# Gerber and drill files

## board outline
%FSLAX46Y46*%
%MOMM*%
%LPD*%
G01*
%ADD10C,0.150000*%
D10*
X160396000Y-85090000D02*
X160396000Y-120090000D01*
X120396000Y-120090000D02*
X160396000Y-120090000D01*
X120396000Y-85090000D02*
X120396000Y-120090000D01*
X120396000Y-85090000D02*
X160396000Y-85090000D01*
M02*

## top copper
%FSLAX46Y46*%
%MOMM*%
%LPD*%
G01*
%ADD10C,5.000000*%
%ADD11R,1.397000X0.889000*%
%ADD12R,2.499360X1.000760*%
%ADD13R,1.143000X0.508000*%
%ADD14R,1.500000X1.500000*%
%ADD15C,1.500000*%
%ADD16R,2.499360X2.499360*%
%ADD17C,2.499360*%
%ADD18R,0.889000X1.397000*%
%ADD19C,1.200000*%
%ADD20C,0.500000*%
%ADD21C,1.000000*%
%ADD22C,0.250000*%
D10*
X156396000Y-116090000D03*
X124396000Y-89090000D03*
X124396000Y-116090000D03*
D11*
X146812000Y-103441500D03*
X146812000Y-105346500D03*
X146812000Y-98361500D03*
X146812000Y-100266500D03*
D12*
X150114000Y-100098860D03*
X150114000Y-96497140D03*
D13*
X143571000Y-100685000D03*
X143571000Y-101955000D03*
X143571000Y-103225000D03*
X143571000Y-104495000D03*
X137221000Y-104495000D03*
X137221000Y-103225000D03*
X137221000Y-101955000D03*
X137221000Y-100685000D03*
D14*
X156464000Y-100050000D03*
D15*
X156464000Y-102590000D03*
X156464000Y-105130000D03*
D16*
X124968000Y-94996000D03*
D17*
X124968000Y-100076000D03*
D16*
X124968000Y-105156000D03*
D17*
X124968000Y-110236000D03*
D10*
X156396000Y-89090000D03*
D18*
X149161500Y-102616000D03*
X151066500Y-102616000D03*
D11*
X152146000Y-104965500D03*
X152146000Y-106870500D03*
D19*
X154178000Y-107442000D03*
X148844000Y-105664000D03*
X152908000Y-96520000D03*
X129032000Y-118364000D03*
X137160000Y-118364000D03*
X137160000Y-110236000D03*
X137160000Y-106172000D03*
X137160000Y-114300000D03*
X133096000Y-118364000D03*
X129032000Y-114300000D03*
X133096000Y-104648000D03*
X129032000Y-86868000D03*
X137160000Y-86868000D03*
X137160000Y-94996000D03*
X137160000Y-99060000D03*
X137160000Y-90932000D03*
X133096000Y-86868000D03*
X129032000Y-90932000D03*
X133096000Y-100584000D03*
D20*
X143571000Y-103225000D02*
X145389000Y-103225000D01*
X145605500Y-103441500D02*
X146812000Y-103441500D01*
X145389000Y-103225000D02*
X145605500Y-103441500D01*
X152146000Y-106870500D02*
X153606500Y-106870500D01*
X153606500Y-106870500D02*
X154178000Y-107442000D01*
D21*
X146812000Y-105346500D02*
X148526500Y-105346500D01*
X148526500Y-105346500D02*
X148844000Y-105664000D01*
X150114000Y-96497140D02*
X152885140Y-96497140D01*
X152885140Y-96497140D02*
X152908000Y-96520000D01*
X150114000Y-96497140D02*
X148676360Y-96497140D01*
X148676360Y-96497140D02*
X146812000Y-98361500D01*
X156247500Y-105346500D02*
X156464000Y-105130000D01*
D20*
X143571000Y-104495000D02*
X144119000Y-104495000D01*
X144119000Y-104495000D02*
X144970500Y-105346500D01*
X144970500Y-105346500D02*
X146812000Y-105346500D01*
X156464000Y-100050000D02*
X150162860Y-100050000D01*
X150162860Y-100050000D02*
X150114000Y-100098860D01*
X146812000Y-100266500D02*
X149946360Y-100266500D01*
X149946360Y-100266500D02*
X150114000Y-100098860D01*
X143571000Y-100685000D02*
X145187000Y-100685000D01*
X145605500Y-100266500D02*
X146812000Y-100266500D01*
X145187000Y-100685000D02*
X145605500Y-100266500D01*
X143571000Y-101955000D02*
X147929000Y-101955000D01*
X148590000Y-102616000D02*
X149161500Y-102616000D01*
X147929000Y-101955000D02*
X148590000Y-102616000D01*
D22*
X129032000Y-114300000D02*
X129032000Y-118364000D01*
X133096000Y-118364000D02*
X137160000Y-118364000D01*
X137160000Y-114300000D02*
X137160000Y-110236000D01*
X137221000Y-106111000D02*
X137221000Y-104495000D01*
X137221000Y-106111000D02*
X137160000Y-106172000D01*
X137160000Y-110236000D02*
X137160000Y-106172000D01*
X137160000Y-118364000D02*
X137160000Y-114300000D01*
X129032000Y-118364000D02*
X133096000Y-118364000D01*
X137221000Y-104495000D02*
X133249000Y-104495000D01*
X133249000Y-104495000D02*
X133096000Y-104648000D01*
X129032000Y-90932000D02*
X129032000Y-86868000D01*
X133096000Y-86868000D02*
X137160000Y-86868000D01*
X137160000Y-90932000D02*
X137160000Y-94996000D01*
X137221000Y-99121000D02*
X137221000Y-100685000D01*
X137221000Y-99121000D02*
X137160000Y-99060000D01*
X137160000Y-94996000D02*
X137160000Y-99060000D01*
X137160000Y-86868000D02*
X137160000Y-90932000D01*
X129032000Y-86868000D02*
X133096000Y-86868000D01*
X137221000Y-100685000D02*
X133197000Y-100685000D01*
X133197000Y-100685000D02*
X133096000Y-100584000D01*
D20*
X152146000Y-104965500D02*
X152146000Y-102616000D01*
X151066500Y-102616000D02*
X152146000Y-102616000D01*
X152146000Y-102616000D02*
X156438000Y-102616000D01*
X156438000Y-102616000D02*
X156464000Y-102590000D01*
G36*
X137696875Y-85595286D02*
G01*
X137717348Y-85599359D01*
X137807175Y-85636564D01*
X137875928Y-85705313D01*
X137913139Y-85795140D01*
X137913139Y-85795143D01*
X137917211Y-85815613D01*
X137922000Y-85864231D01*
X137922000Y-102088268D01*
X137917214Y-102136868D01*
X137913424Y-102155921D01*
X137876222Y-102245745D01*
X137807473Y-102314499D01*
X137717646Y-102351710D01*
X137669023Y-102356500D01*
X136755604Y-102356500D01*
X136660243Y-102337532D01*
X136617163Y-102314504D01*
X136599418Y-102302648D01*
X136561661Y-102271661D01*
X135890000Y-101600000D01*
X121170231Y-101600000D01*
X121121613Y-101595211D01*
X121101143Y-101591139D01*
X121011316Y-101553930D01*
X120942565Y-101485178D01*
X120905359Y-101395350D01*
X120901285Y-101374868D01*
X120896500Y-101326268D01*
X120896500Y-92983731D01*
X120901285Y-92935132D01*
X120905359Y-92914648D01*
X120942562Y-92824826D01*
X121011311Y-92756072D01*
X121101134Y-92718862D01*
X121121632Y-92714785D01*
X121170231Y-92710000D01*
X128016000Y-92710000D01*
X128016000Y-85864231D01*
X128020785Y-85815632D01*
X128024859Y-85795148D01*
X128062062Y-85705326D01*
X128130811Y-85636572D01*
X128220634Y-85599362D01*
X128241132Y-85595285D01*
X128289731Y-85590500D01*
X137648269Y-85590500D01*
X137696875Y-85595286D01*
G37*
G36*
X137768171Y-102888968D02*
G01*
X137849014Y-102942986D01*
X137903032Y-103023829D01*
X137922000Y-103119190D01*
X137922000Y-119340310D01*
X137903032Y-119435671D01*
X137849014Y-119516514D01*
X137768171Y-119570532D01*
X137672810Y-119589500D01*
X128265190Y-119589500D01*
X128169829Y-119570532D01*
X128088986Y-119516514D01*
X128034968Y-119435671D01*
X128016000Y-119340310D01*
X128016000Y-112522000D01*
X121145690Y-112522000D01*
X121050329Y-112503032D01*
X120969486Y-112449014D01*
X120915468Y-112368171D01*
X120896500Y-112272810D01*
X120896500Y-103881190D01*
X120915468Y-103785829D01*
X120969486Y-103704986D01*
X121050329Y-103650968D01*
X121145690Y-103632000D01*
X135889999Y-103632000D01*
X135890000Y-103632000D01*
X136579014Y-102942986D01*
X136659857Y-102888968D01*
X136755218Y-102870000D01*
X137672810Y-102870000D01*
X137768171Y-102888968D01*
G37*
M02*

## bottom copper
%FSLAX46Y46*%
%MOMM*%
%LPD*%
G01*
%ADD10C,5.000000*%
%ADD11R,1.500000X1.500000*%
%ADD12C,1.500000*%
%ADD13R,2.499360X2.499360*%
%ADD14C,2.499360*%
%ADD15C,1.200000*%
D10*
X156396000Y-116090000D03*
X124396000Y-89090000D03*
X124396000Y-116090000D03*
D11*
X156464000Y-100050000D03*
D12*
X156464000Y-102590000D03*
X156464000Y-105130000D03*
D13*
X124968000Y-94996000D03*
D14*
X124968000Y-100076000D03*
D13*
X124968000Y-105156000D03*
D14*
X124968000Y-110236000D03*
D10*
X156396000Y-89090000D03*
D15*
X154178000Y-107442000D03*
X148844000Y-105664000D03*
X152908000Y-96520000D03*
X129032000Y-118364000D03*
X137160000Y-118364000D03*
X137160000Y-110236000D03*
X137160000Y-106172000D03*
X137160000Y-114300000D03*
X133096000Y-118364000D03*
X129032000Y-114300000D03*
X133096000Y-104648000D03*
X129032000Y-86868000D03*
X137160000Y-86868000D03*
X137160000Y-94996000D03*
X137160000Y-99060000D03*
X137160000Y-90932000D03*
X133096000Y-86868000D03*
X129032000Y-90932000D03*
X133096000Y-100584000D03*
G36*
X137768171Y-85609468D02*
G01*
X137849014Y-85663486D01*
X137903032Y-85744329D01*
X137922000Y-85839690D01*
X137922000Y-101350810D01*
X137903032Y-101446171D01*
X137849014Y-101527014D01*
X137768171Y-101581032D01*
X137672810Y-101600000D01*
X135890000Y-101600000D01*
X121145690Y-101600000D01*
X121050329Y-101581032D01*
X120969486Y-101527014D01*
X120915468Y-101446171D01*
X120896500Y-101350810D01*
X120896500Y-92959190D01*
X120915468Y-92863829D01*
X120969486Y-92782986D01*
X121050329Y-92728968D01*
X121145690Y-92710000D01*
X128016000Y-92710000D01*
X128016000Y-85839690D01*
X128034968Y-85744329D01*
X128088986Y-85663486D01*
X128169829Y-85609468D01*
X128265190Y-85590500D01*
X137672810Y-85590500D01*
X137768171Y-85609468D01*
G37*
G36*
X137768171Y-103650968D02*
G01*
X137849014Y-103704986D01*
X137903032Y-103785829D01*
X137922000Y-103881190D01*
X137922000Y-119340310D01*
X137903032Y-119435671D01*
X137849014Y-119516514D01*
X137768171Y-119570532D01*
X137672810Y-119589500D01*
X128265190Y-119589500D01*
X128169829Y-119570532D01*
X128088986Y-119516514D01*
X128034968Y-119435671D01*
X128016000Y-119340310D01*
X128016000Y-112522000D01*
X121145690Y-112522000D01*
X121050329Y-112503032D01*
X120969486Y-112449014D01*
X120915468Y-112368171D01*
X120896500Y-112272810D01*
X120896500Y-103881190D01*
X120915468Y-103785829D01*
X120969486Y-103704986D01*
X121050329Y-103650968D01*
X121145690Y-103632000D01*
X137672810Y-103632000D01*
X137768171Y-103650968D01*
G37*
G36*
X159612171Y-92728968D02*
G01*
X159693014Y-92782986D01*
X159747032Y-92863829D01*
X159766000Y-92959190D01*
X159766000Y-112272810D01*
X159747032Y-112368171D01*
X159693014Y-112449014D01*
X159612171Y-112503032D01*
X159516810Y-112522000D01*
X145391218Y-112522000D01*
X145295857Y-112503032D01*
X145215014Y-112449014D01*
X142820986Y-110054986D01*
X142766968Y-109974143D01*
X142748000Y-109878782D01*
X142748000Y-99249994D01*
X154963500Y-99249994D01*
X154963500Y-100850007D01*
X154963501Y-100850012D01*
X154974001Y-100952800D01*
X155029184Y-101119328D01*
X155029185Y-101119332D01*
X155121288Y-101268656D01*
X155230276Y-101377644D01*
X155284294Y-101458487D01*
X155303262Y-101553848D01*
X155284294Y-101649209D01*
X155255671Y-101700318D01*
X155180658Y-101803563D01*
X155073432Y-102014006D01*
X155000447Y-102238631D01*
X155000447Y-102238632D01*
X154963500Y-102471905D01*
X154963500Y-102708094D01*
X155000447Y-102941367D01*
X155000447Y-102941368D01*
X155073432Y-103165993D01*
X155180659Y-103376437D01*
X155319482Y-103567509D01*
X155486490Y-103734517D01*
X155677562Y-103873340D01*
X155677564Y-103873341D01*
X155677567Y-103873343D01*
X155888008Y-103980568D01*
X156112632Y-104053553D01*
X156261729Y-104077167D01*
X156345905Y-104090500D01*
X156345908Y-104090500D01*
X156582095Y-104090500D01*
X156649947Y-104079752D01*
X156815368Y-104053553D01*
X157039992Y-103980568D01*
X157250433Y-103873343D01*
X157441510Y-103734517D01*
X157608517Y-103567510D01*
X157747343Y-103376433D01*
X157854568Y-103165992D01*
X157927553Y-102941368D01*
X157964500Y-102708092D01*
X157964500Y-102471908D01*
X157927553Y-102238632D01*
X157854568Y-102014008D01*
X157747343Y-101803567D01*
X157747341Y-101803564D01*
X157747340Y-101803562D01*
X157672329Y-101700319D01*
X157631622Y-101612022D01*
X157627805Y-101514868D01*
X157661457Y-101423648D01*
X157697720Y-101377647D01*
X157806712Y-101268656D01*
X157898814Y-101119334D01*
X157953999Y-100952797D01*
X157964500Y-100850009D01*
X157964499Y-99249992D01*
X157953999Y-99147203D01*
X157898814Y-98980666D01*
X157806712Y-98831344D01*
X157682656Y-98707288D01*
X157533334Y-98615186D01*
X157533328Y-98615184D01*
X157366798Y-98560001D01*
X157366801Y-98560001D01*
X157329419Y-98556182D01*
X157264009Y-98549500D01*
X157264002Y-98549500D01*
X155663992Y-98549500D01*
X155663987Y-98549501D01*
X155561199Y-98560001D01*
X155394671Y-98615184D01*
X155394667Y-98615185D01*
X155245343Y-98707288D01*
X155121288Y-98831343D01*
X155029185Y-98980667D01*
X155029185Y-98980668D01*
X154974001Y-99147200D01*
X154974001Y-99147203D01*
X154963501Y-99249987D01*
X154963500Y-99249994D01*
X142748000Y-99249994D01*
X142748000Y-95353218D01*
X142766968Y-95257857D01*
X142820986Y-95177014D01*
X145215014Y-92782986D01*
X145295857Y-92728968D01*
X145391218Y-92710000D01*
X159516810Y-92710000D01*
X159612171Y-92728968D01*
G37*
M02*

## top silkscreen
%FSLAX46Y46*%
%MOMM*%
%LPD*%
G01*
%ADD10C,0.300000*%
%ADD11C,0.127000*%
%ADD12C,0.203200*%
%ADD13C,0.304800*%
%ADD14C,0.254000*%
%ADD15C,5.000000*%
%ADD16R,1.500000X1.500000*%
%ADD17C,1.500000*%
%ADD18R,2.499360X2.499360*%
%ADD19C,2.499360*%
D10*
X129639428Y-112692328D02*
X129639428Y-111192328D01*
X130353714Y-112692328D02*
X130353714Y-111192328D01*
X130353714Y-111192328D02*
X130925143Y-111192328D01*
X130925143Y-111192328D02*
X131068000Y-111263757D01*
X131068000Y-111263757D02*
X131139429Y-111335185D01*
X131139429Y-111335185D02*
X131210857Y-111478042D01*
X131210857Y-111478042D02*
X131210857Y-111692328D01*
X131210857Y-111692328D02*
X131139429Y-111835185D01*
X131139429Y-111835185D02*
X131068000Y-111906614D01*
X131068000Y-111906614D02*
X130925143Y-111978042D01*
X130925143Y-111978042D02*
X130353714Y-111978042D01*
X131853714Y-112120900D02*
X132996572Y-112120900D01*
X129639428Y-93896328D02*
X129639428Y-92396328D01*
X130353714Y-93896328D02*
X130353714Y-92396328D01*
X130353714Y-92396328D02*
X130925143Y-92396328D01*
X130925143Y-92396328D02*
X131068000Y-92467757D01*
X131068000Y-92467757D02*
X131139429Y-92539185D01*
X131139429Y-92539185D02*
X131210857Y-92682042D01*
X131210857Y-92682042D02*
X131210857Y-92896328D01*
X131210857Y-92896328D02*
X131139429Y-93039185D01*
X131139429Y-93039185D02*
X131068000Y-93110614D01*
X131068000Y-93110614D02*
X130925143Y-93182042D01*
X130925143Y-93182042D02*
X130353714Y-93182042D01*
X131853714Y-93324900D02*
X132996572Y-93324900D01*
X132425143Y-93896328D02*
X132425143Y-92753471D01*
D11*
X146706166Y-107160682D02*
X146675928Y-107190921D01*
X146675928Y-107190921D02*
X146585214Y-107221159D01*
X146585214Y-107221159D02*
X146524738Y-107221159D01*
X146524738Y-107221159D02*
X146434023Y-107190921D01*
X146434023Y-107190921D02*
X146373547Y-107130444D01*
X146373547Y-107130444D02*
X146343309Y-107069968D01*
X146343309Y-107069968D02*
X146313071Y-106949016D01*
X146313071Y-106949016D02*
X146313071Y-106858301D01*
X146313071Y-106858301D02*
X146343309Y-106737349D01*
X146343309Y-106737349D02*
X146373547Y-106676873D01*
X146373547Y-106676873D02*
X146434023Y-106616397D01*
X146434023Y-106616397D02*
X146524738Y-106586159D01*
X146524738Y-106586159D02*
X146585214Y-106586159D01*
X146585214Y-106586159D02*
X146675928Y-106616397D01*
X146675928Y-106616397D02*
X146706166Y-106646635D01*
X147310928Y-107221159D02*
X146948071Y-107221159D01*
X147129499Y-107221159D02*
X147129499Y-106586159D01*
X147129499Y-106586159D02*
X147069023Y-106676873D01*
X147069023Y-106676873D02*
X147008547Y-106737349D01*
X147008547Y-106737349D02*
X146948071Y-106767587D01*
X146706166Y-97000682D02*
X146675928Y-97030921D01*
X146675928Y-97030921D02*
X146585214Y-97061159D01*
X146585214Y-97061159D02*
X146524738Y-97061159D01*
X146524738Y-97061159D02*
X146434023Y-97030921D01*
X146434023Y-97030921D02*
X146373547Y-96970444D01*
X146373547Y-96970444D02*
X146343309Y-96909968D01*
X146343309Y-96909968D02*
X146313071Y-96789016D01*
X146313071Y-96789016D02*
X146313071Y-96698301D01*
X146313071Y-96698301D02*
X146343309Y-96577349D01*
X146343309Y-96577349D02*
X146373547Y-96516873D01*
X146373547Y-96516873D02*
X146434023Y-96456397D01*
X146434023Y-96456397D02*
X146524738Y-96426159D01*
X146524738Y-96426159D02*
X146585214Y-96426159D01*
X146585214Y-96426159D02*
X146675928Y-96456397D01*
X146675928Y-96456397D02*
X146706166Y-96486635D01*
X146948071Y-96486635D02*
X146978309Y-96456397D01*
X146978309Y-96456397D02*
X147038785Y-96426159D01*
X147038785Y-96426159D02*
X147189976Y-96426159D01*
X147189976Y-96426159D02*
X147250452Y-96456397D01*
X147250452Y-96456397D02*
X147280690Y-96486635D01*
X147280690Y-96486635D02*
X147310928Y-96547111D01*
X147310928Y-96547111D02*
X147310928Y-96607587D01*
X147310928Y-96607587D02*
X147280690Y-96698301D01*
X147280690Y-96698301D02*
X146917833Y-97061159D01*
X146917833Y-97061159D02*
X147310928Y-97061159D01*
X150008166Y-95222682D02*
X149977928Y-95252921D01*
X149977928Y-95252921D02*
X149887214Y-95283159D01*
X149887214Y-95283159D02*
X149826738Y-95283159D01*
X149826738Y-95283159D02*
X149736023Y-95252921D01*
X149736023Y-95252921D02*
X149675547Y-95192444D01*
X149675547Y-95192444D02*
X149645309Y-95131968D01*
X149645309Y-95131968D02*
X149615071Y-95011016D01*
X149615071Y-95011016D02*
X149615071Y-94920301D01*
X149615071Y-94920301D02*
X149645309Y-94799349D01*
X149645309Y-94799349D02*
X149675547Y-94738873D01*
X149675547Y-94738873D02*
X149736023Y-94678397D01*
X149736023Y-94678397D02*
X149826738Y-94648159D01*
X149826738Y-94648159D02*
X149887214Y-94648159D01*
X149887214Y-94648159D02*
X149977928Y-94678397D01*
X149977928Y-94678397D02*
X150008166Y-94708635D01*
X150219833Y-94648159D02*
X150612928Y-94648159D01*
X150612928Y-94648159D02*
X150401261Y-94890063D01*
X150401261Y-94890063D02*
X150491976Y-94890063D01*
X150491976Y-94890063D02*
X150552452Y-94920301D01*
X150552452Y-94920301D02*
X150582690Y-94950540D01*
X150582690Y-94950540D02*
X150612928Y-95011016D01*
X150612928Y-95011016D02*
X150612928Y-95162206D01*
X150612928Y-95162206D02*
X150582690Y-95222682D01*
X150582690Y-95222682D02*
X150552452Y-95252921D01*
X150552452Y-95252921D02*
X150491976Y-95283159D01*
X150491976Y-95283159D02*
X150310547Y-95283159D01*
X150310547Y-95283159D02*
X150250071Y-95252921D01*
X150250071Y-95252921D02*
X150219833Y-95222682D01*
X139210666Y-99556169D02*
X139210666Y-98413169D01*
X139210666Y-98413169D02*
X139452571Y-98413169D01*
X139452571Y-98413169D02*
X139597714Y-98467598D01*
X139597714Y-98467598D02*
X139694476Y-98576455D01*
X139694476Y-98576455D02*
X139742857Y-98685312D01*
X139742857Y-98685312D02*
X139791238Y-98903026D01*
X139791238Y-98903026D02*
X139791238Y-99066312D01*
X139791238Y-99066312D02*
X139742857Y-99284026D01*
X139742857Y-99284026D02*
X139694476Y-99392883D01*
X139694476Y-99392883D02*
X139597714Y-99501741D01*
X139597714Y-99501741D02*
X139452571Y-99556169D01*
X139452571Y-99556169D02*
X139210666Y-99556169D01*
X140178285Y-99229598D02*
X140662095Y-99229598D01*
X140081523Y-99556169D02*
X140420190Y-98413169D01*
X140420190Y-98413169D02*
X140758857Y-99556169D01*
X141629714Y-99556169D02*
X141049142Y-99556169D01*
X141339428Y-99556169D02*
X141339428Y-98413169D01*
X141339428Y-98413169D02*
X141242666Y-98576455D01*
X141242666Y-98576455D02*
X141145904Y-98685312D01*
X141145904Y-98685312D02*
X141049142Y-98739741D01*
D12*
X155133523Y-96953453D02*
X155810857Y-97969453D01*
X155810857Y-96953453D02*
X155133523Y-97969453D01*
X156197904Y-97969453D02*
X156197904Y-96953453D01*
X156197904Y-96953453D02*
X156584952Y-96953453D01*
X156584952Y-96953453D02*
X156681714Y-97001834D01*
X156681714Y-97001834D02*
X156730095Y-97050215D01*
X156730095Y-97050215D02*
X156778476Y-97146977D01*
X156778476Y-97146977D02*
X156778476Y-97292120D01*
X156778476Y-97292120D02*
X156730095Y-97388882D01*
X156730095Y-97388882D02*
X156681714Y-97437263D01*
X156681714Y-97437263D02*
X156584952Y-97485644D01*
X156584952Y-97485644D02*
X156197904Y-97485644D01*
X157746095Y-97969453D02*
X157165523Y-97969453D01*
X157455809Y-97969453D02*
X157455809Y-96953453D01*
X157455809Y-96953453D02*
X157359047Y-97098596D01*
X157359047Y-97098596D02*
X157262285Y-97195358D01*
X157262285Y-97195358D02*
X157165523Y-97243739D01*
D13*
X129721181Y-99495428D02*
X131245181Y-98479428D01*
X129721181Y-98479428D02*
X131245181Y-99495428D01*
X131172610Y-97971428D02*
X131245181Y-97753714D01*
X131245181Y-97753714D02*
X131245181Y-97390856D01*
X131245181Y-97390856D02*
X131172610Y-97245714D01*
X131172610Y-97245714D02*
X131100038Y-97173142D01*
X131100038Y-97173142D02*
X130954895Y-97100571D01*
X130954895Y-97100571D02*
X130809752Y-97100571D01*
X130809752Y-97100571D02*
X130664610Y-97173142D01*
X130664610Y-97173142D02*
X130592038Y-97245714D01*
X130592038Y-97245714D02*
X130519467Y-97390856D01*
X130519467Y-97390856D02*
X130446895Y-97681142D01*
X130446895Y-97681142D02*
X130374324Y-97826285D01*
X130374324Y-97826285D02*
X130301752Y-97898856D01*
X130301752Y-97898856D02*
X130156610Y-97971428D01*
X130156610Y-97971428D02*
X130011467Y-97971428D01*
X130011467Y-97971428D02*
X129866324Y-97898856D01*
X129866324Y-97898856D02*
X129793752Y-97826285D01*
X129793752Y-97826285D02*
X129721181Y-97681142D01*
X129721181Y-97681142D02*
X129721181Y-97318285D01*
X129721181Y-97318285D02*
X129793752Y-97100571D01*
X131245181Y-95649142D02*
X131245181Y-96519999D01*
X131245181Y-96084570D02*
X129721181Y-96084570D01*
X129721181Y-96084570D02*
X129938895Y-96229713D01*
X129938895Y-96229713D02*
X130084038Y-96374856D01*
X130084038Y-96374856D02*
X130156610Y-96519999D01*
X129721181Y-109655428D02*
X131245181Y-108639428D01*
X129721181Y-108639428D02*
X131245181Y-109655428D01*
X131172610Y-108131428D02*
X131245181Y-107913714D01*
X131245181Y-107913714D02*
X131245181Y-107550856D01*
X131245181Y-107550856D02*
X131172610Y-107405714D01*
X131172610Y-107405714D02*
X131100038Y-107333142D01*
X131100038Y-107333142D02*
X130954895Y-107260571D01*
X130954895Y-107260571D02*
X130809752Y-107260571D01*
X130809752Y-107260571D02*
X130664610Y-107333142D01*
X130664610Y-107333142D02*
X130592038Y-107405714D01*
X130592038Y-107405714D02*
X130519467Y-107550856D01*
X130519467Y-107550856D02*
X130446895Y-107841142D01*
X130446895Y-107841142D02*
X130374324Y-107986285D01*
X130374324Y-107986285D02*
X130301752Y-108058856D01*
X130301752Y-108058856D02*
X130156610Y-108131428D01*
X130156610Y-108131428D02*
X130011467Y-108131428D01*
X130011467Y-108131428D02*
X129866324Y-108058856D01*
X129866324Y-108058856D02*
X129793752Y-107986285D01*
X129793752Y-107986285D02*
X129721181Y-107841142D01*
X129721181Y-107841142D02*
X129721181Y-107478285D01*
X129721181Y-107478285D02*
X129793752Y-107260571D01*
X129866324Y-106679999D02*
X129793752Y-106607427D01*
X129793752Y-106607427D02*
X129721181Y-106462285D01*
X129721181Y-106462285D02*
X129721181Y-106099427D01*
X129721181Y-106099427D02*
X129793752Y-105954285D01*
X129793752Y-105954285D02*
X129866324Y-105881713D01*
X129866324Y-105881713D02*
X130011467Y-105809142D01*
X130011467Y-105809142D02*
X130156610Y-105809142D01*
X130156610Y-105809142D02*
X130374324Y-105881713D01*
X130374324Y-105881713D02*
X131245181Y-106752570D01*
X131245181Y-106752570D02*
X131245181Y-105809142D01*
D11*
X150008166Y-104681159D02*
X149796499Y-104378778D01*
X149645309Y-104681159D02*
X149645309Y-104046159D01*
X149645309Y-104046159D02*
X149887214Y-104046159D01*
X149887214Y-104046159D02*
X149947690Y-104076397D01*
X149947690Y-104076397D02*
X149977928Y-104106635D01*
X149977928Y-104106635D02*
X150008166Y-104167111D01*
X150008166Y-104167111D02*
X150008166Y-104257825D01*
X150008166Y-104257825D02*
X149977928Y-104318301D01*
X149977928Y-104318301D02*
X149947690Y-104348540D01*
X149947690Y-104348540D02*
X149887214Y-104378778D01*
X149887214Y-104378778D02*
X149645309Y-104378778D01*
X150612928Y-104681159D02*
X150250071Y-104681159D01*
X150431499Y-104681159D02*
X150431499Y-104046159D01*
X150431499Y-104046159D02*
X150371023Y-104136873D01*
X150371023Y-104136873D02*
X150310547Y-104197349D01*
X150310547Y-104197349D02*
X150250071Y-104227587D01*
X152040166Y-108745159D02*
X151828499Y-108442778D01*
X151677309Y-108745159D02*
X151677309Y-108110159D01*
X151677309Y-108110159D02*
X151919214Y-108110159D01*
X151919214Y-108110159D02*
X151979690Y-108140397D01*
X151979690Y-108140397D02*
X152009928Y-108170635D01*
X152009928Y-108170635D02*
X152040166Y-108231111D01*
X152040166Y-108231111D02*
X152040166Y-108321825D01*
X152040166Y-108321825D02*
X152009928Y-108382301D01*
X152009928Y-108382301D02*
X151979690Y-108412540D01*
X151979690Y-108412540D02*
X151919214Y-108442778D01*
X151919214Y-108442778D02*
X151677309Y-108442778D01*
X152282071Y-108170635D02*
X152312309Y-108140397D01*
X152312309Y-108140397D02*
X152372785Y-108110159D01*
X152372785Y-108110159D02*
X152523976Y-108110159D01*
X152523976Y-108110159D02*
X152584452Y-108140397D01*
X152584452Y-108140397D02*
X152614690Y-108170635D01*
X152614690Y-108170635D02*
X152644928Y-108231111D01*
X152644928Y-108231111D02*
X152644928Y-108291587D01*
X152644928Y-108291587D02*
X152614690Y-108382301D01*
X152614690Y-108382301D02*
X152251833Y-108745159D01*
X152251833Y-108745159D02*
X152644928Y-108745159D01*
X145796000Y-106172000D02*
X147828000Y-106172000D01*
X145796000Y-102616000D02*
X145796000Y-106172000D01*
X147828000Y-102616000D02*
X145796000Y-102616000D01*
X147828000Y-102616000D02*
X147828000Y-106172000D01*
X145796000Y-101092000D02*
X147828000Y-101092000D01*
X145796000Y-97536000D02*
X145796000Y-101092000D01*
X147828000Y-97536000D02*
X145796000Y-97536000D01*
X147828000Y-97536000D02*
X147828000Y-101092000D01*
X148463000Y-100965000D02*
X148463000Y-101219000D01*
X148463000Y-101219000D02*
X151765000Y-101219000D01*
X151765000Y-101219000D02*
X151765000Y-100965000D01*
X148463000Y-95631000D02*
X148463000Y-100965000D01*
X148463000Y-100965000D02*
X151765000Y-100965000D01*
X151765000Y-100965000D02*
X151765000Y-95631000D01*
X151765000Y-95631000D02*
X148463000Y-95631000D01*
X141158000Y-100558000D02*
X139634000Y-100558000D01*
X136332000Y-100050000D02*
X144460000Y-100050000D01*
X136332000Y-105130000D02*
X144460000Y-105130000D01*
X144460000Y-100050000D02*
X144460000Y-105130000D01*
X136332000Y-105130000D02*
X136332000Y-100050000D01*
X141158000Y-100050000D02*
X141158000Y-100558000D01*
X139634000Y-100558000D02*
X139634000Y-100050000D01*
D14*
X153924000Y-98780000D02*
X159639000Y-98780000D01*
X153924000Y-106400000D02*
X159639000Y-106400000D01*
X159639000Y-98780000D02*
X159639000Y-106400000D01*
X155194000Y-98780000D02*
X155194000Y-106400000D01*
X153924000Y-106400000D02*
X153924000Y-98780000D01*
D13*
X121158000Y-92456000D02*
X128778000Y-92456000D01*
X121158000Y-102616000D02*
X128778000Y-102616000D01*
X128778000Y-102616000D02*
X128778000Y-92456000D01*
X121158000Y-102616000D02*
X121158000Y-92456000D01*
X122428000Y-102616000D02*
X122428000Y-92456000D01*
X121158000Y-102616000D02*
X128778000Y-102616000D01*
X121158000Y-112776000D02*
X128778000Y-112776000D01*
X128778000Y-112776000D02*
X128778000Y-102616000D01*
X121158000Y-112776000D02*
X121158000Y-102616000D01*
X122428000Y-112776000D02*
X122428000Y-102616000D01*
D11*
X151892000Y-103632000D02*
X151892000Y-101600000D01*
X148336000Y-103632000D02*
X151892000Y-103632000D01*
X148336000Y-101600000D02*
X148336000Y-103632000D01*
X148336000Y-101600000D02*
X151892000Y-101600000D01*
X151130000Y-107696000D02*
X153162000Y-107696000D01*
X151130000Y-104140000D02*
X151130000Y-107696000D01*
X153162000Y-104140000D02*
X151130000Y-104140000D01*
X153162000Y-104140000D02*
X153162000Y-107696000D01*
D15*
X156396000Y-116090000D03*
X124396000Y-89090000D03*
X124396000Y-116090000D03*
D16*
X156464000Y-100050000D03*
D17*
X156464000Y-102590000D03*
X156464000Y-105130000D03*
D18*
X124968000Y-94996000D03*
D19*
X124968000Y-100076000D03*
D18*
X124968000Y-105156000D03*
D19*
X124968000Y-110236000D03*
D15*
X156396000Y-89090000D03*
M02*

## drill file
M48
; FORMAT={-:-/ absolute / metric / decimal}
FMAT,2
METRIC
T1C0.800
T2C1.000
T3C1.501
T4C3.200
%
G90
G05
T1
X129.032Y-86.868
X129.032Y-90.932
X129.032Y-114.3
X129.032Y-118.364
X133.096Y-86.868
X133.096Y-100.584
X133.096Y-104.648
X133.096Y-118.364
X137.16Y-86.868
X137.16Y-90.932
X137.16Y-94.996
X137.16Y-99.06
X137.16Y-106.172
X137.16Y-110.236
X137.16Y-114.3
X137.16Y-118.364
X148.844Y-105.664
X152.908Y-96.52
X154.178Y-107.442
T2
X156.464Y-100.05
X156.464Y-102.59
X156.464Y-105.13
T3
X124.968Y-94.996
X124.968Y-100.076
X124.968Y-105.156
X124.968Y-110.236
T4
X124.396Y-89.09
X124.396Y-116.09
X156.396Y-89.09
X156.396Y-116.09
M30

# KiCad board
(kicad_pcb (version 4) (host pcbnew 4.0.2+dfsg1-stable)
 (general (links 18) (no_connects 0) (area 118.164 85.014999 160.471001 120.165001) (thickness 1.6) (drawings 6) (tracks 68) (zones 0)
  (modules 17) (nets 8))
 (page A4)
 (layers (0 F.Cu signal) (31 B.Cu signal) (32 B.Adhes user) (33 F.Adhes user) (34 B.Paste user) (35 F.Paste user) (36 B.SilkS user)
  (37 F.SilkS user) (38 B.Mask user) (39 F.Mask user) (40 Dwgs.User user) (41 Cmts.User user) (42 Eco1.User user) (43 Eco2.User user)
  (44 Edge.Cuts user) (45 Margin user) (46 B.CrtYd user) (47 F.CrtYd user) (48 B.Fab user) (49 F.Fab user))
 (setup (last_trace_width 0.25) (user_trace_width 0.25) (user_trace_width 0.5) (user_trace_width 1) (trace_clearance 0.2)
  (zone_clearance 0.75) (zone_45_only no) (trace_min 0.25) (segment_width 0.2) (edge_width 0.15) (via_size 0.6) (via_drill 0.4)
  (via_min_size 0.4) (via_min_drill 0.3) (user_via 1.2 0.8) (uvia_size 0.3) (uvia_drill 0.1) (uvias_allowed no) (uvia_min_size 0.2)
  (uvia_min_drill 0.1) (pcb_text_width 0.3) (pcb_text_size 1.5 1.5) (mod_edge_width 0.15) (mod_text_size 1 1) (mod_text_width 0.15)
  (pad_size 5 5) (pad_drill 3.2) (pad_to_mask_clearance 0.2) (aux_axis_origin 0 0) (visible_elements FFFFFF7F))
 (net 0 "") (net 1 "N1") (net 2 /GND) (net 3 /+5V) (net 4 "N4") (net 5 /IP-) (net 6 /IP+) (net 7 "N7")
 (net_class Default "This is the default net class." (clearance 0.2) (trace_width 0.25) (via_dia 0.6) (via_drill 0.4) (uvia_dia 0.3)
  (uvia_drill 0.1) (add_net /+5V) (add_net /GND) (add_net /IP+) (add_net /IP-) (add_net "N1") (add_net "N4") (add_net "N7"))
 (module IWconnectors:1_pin (layer F.Cu) (at 124.968 113.284)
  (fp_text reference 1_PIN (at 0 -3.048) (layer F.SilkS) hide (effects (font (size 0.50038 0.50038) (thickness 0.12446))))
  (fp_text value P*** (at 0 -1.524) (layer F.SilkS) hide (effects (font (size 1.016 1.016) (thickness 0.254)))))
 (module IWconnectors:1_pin (layer F.Cu) (at 124.968 89.916)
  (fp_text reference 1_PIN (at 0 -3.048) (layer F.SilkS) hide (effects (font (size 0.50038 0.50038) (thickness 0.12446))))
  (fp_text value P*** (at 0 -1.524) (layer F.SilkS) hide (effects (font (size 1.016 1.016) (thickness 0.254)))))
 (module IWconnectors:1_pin (layer B.Cu) (at 124.968 115.316)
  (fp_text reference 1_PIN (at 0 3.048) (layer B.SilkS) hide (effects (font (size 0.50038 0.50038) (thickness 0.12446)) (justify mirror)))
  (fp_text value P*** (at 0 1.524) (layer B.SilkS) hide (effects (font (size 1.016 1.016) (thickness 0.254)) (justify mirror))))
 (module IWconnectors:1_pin (layer B.Cu) (at 124.968 115.316)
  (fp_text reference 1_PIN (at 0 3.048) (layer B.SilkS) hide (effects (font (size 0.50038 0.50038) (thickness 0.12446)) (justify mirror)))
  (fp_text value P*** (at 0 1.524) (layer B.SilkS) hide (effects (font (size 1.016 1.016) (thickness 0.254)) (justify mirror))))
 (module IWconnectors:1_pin (layer F.Cu) (at 155.448 114.554)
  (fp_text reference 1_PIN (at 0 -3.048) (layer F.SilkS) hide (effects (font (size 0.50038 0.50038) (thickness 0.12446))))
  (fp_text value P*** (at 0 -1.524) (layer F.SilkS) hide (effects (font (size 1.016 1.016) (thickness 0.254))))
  (pad 1 thru_hole circle (at 0.948 1.536) (size 5 5) (drill 3.2) (layers *.Cu *.Mask F.SilkS)))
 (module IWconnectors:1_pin (layer F.Cu) (at 124.968 89.916)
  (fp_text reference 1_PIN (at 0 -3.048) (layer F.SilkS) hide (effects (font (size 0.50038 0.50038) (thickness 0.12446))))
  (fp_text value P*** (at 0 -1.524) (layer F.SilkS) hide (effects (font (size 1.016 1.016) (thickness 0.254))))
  (pad 1 thru_hole circle (at -0.572 -0.826) (size 5 5) (drill 3.2) (layers *.Cu *.Mask F.SilkS)))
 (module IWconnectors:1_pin (layer F.Cu) (at 124.968 113.284)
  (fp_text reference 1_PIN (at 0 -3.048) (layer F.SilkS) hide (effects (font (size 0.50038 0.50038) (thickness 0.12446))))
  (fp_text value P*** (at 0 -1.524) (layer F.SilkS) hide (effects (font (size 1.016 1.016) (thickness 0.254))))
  (pad 1 thru_hole circle (at -0.572 2.806) (size 5 5) (drill 3.2) (layers *.Cu *.Mask F.SilkS)))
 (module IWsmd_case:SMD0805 (layer F.Cu) (at 146.812 104.394 270)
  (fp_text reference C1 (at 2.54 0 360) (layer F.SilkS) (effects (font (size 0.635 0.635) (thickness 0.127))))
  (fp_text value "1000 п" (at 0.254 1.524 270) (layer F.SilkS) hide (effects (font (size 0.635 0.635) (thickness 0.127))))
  (fp_line (start 1.778 1.016) (end 1.778 -1.016) (layer F.SilkS) (width 0.127))
  (fp_line (start -1.778 1.016) (end 1.778 1.016) (layer F.SilkS) (width 0.127))
  (fp_line (start -1.778 -1.016) (end -1.778 1.016) (layer F.SilkS) (width 0.127))
  (fp_line (start -1.778 -1.016) (end 1.778 -1.016) (layer F.SilkS) (width 0.127))
  (pad 1 smd rect (at -0.9525 0 270) (size 0.889 1.397) (layers F.Cu F.Paste F.Mask) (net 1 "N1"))
  (pad 2 smd rect (at 0.9525 0 270) (size 0.889 1.397) (layers F.Cu F.Paste F.Mask) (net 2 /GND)))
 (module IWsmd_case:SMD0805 (layer F.Cu) (at 146.812 99.314 270)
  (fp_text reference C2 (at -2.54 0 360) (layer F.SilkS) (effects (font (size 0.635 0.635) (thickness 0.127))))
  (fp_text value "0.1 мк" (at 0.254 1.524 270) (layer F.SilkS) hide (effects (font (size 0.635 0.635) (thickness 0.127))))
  (fp_line (start 1.778 1.016) (end 1.778 -1.016) (layer F.SilkS) (width 0.127))
  (fp_line (start -1.778 1.016) (end 1.778 1.016) (layer F.SilkS) (width 0.127))
  (fp_line (start -1.778 -1.016) (end -1.778 1.016) (layer F.SilkS) (width 0.127))
  (fp_line (start -1.778 -1.016) (end 1.778 -1.016) (layer F.SilkS) (width 0.127))
  (pad 1 smd rect (at -0.9525 0 270) (size 0.889 1.397) (layers F.Cu F.Paste F.Mask) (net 2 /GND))
  (pad 2 smd rect (at 0.9525 0 270) (size 0.889 1.397) (layers F.Cu F.Paste F.Mask) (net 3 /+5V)))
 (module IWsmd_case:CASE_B (layer F.Cu) (at 150.114 98.298 90)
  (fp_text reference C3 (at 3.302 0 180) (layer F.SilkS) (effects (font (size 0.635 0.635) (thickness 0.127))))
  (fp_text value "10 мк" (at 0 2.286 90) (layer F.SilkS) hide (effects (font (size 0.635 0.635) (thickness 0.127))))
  (fp_line (start -2.667 -1.651) (end -2.921 -1.651) (layer F.SilkS) (width 0.127))
  (fp_line (start -2.921 -1.651) (end -2.921 1.651) (layer F.SilkS) (width 0.127))
  (fp_line (start -2.921 1.651) (end -2.667 1.651) (layer F.SilkS) (width 0.127))
  (fp_line (start 2.667 -1.651) (end -2.667 -1.651) (layer F.SilkS) (width 0.127))
  (fp_line (start -2.667 -1.651) (end -2.667 1.651) (layer F.SilkS) (width 0.127))
  (fp_line (start -2.667 1.651) (end 2.667 1.651) (layer F.SilkS) (width 0.127))
  (fp_line (start 2.667 1.651) (end 2.667 -1.651) (layer F.SilkS) (width 0.127))
  (pad 1 smd rect (at -1.80086 0 90) (size 1.00076 2.49936) (layers F.Cu F.Paste F.Mask) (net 3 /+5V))
  (pad 2 smd rect (at 1.80086 0 90) (size 1.00076 2.49936) (layers F.Cu F.Paste F.Mask) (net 2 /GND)))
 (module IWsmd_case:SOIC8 (layer F.Cu) (at 140.396 102.59 270)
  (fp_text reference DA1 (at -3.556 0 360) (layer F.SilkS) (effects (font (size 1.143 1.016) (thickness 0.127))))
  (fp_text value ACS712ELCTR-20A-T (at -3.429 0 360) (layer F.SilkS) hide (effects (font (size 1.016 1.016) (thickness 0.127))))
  (fp_line (start -2.032 -0.762) (end -2.032 0.762) (layer F.SilkS) (width 0.127))
  (fp_line (start -2.54 4.064) (end -2.54 -4.064) (layer F.SilkS) (width 0.127))
  (fp_line (start 2.54 4.064) (end 2.54 -4.064) (layer F.SilkS) (width 0.127))
  (fp_line (start -2.54 -4.064) (end 2.54 -4.064) (layer F.SilkS) (width 0.127))
  (fp_line (start 2.54 4.064) (end -2.54 4.064) (layer F.SilkS) (width 0.127))
  (fp_line (start -2.54 -0.762) (end -2.032 -0.762) (layer F.SilkS) (width 0.127))
  (fp_line (start -2.032 0.762) (end -2.54 0.762) (layer F.SilkS) (width 0.127))
  (pad 8 smd rect (at -1.905 -3.175 270) (size 0.508 1.143) (layers F.Cu F.Paste F.Mask) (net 3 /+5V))
  (pad 7 smd rect (at -0.635 -3.175 270) (size 0.508 1.143) (layers F.Cu F.Paste F.Mask) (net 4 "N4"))
  (pad 6 smd rect (at 0.635 -3.175 270) (size 0.508 1.143) (layers F.Cu F.Paste F.Mask) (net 1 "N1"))
  (pad 5 smd rect (at 1.905 -3.175 270) (size 0.508 1.143) (layers F.Cu F.Paste F.Mask) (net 2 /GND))
  (pad 4 smd rect (at 1.905 3.175 270) (size 0.508 1.143) (layers F.Cu F.Paste F.Mask) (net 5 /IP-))
  (pad 3 smd rect (at 0.635 3.175 270) (size 0.508 1.143) (layers F.Cu F.Paste F.Mask) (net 5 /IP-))
  (pad 2 smd rect (at -0.635 3.175 270) (size 0.508 1.143) (layers F.Cu F.Paste F.Mask) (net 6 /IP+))
  (pad 1 smd rect (at -1.905 3.175 270) (size 0.508 1.143) (layers F.Cu F.Paste F.Mask) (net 6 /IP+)))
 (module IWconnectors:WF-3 (layer F.Cu) (at 156.464 102.59 270)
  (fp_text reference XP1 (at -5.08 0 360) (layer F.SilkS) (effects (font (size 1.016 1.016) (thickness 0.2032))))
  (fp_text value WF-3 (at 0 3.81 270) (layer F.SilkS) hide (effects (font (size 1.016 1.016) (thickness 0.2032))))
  (fp_line (start -3.81 2.54) (end -3.81 -3.175) (layer F.SilkS) (width 0.254))
  (fp_line (start 3.81 2.54) (end 3.81 -3.175) (layer F.SilkS) (width 0.254))
  (fp_line (start -3.81 -3.175) (end 3.81 -3.175) (layer F.SilkS) (width 0.254))
  (fp_line (start -3.81 1.27) (end 3.81 1.27) (layer F.SilkS) (width 0.254))
  (fp_line (start 3.81 2.54) (end -3.81 2.54) (layer F.SilkS) (width 0.254))
  (pad 1 thru_hole rect (at -2.54 0 270) (size 1.5 1.5) (drill 1) (layers *.Cu *.Mask F.SilkS) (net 3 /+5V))
  (pad 2 thru_hole circle (at 0 0 270) (size 1.5 1.5) (drill 1) (layers *.Cu *.Mask F.SilkS) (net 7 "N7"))
  (pad 3 thru_hole circle (at 2.54 0 270) (size 1.5 1.5) (drill 1) (layers *.Cu *.Mask F.SilkS) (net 2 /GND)))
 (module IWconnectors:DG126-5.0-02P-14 (layer F.Cu) (at 124.968 97.536 270)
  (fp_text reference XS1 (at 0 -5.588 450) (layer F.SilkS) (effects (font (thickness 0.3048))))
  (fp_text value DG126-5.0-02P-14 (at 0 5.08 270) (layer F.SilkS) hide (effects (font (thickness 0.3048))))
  (fp_line (start -5.08 3.81) (end -5.08 -3.81) (layer F.SilkS) (width 0.3048))
  (fp_line (start 5.08 3.81) (end 5.08 -3.81) (layer F.SilkS) (width 0.3048))
  (fp_line (start 5.08 -3.81) (end -5.08 -3.81) (layer F.SilkS) (width 0.3048))
  (fp_line (start 5.08 3.81) (end -5.08 3.81) (layer F.SilkS) (width 0.3048))
  (fp_line (start 5.08 2.54) (end -5.08 2.54) (layer F.SilkS) (width 0.3048))
  (pad 1 thru_hole rect (at -2.54 0 270) (size 2.49936 2.49936) (drill 1.50114) (layers *.Cu *.Mask F.SilkS) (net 6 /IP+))
  (pad 2 thru_hole circle (at 2.54 0 270) (size 2.49936 2.49936) (drill 1.50114) (layers *.Cu *.Mask F.SilkS) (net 6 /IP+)))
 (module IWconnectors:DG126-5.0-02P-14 (layer F.Cu) (at 124.968 107.696 270)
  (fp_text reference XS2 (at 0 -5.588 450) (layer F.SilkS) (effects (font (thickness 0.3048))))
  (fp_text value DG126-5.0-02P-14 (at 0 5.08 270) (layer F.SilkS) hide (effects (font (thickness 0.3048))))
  (fp_line (start -5.08 3.81) (end -5.08 -3.81) (layer F.SilkS) (width 0.3048))
  (fp_line (start 5.08 3.81) (end 5.08 -3.81) (layer F.SilkS) (width 0.3048))
  (fp_line (start 5.08 -3.81) (end -5.08 -3.81) (layer F.SilkS) (width 0.3048))
  (fp_line (start 5.08 3.81) (end -5.08 3.81) (layer F.SilkS) (width 0.3048))
  (fp_line (start 5.08 2.54) (end -5.08 2.54) (layer F.SilkS) (width 0.3048))
  (pad 1 thru_hole rect (at -2.54 0 270) (size 2.49936 2.49936) (drill 1.50114) (layers *.Cu *.Mask F.SilkS) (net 5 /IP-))
  (pad 2 thru_hole circle (at 2.54 0 270) (size 2.49936 2.49936) (drill 1.50114) (layers *.Cu *.Mask F.SilkS) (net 5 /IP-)))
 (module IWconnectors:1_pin (layer F.Cu) (at 153.416 89.916)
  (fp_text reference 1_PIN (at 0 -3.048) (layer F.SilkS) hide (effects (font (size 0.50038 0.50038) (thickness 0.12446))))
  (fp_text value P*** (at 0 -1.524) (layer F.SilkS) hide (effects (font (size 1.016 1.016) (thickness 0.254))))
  (pad 1 thru_hole circle (at 2.98 -0.826) (size 5 5) (drill 3.2) (layers *.Cu *.Mask F.SilkS)))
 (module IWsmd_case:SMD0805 (layer F.Cu) (at 150.114 102.616)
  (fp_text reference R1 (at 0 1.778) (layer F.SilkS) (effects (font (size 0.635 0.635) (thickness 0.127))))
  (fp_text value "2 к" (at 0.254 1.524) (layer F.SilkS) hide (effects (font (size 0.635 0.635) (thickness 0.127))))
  (fp_line (start 1.778 1.016) (end 1.778 -1.016) (layer F.SilkS) (width 0.127))
  (fp_line (start -1.778 1.016) (end 1.778 1.016) (layer F.SilkS) (width 0.127))
  (fp_line (start -1.778 -1.016) (end -1.778 1.016) (layer F.SilkS) (width 0.127))
  (fp_line (start -1.778 -1.016) (end 1.778 -1.016) (layer F.SilkS) (width 0.127))
  (pad 1 smd rect (at -0.9525 0) (size 0.889 1.397) (layers F.Cu F.Paste F.Mask) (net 4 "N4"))
  (pad 2 smd rect (at 0.9525 0) (size 0.889 1.397) (layers F.Cu F.Paste F.Mask) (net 7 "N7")))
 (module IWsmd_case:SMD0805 (layer F.Cu) (at 152.146 105.918 270)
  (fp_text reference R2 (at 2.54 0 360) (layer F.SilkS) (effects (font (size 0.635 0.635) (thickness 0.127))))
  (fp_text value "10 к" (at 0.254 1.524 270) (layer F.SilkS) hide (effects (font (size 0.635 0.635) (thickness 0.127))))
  (fp_line (start 1.778 1.016) (end 1.778 -1.016) (layer F.SilkS) (width 0.127))
  (fp_line (start -1.778 1.016) (end 1.778 1.016) (layer F.SilkS) (width 0.127))
  (fp_line (start -1.778 -1.016) (end -1.778 1.016) (layer F.SilkS) (width 0.127))
  (fp_line (start -1.778 -1.016) (end 1.778 -1.016) (layer F.SilkS) (width 0.127))
  (pad 1 smd rect (at -0.9525 0 270) (size 0.889 1.397) (layers F.Cu F.Paste F.Mask) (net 7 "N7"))
  (pad 2 smd rect (at 0.9525 0 270) (size 0.889 1.397) (layers F.Cu F.Paste F.Mask) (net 2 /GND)))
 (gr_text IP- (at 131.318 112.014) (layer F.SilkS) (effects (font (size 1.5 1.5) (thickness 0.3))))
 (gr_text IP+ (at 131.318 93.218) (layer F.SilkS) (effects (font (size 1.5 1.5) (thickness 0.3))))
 (gr_line (start 160.396 85.09) (end 160.396 120.09) (angle 90) (layer Edge.Cuts) (width 0.15))
 (gr_line (start 120.396 120.09) (end 160.396 120.09) (angle 90) (layer Edge.Cuts) (width 0.15))
 (gr_line (start 120.396 85.09) (end 120.396 120.09) (angle 90) (layer Edge.Cuts) (width 0.15))
 (gr_line (start 120.396 85.09) (end 160.396 85.09) (angle 90) (layer Edge.Cuts) (width 0.15))
 (segment (start 143.571 103.225) (end 145.389 103.225) (width 0.5) (layer F.Cu) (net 1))
 (segment (start 145.6055 103.4415) (end 146.812 103.4415) (width 0.5) (layer F.Cu) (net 1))
 (segment (start 145.389 103.225) (end 145.6055 103.4415) (width 0.5) (layer F.Cu) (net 1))
 (segment (start 152.146 106.8705) (end 153.6065 106.8705) (width 0.5) (layer F.Cu) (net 2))
 (via (at 154.178 107.442) (size 1.2) (drill 0.8) (layers F.Cu B.Cu) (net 2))
 (segment (start 153.6065 106.8705) (end 154.178 107.442) (width 0.5) (layer F.Cu) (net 2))
 (segment (start 146.812 105.3465) (end 148.5265 105.3465) (width 1) (layer F.Cu) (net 2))
 (via (at 148.844 105.664) (size 1.2) (drill 0.8) (layers F.Cu B.Cu) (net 2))
 (segment (start 148.5265 105.3465) (end 148.844 105.664) (width 1) (layer F.Cu) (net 2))
 (segment (start 150.114 96.49714) (end 152.88514 96.49714) (width 1) (layer F.Cu) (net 2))
 (via (at 152.908 96.52) (size 1.2) (drill 0.8) (layers F.Cu B.Cu) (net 2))
 (segment (start 152.88514 96.49714) (end 152.908 96.52) (width 1) (layer F.Cu) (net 2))
 (segment (start 150.114 96.49714) (end 148.67636 96.49714) (width 1) (layer F.Cu) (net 2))
 (segment (start 148.67636 96.49714) (end 146.812 98.3615) (width 1) (layer F.Cu) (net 2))
 (segment (start 156.2475 105.3465) (end 156.464 105.13) (width 1) (layer F.Cu) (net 2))
 (segment (start 143.571 104.495) (end 144.119 104.495) (width 0.5) (layer F.Cu) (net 2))
 (segment (start 144.119 104.495) (end 144.9705 105.3465) (width 0.5) (layer F.Cu) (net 2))
 (segment (start 144.9705 105.3465) (end 146.812 105.3465) (width 0.5) (layer F.Cu) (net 2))
 (segment (start 156.464 100.05) (end 150.16286 100.05) (width 0.5) (layer F.Cu) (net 3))
 (segment (start 150.16286 100.05) (end 150.114 100.09886) (width 0.5) (layer F.Cu) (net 3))
 (segment (start 146.812 100.2665) (end 149.94636 100.2665) (width 0.5) (layer F.Cu) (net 3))
 (segment (start 149.94636 100.2665) (end 150.114 100.09886) (width 0.5) (layer F.Cu) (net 3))
 (segment (start 143.571 100.685) (end 145.187 100.685) (width 0.5) (layer F.Cu) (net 3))
 (segment (start 145.6055 100.2665) (end 146.812 100.2665) (width 0.5) (layer F.Cu) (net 3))
 (segment (start 145.187 100.685) (end 145.6055 100.2665) (width 0.5) (layer F.Cu) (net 3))
 (segment (start 143.571 101.955) (end 147.929 101.955) (width 0.5) (layer F.Cu) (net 4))
 (segment (start 148.59 102.616) (end 149.1615 102.616) (width 0.5) (layer F.Cu) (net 4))
 (segment (start 147.929 101.955) (end 148.59 102.616) (width 0.5) (layer F.Cu) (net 4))
 (segment (start 129.032 114.3) (end 129.032 118.364) (width 0.25) (layer F.Cu) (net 5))
 (via (at 129.032 118.364) (size 1.2) (drill 0.8) (layers F.Cu B.Cu) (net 5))
 (segment (start 133.096 118.364) (end 137.16 118.364) (width 0.25) (layer F.Cu) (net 5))
 (via (at 137.16 118.364) (size 1.2) (drill 0.8) (layers F.Cu B.Cu) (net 5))
 (segment (start 137.16 114.3) (end 137.16 110.236) (width 0.25) (layer F.Cu) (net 5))
 (via (at 137.16 110.236) (size 1.2) (drill 0.8) (layers F.Cu B.Cu) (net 5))
 (segment (start 137.221 106.111) (end 137.221 104.495) (width 0.25) (layer F.Cu) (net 5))
 (via (at 137.16 106.172) (size 1.2) (drill 0.8) (layers F.Cu B.Cu) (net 5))
 (segment (start 137.221 106.111) (end 137.16 106.172) (width 0.25) (layer F.Cu) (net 5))
 (segment (start 137.16 110.236) (end 137.16 106.172) (width 0.25) (layer F.Cu) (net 5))
 (via (at 137.16 114.3) (size 1.2) (drill 0.8) (layers F.Cu B.Cu) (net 5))
 (segment (start 137.16 118.364) (end 137.16 114.3) (width 0.25) (layer F.Cu) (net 5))
 (via (at 133.096 118.364) (size 1.2) (drill 0.8) (layers F.Cu B.Cu) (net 5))
 (segment (start 129.032 118.364) (end 133.096 118.364) (width 0.25) (layer F.Cu) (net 5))
 (via (at 129.032 114.3) (size 1.2) (drill 0.8) (layers F.Cu B.Cu) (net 5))
 (segment (start 137.221 104.495) (end 133.249 104.495) (width 0.25) (layer F.Cu) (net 5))
 (via (at 133.096 104.648) (size 1.2) (drill 0.8) (layers F.Cu B.Cu) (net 5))
 (segment (start 133.249 104.495) (end 133.096 104.648) (width 0.25) (layer F.Cu) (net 5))
 (segment (start 129.032 90.932) (end 129.032 86.868) (width 0.25) (layer F.Cu) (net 6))
 (via (at 129.032 86.868) (size 1.2) (drill 0.8) (layers F.Cu B.Cu) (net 6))
 (segment (start 133.096 86.868) (end 137.16 86.868) (width 0.25) (layer F.Cu) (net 6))
 (via (at 137.16 86.868) (size 1.2) (drill 0.8) (layers F.Cu B.Cu) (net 6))
 (segment (start 137.16 90.932) (end 137.16 94.996) (width 0.25) (layer F.Cu) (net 6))
 (via (at 137.16 94.996) (size 1.2) (drill 0.8) (layers F.Cu B.Cu) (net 6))
 (segment (start 137.221 99.121) (end 137.221 100.685) (width 0.25) (layer F.Cu) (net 6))
 (via (at 137.16 99.06) (size 1.2) (drill 0.8) (layers F.Cu B.Cu) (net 6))
 (segment (start 137.221 99.121) (end 137.16 99.06) (width 0.25) (layer F.Cu) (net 6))
 (segment (start 137.16 94.996) (end 137.16 99.06) (width 0.25) (layer F.Cu) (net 6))
 (via (at 137.16 90.932) (size 1.2) (drill 0.8) (layers F.Cu B.Cu) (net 6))
 (segment (start 137.16 86.868) (end 137.16 90.932) (width 0.25) (layer F.Cu) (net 6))
 (via (at 133.096 86.868) (size 1.2) (drill 0.8) (layers F.Cu B.Cu) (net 6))
 (segment (start 129.032 86.868) (end 133.096 86.868) (width 0.25) (layer F.Cu) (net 6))
 (via (at 129.032 90.932) (size 1.2) (drill 0.8) (layers F.Cu B.Cu) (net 6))
 (segment (start 137.221 100.685) (end 133.197 100.685) (width 0.25) (layer F.Cu) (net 6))
 (via (at 133.096 100.584) (size 1.2) (drill 0.8) (layers F.Cu B.Cu) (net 6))
 (segment (start 133.197 100.685) (end 133.096 100.584) (width 0.25) (layer F.Cu) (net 6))
 (segment (start 152.146 104.9655) (end 152.146 102.616) (width 0.5) (layer F.Cu) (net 7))
 (segment (start 151.0665 102.616) (end 152.146 102.616) (width 0.5) (layer F.Cu) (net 7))
 (segment (start 152.146 102.616) (end 156.438 102.616) (width 0.5) (layer F.Cu) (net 7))
 (segment (start 156.438 102.616) (end 156.464 102.59) (width 0.5) (layer F.Cu) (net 7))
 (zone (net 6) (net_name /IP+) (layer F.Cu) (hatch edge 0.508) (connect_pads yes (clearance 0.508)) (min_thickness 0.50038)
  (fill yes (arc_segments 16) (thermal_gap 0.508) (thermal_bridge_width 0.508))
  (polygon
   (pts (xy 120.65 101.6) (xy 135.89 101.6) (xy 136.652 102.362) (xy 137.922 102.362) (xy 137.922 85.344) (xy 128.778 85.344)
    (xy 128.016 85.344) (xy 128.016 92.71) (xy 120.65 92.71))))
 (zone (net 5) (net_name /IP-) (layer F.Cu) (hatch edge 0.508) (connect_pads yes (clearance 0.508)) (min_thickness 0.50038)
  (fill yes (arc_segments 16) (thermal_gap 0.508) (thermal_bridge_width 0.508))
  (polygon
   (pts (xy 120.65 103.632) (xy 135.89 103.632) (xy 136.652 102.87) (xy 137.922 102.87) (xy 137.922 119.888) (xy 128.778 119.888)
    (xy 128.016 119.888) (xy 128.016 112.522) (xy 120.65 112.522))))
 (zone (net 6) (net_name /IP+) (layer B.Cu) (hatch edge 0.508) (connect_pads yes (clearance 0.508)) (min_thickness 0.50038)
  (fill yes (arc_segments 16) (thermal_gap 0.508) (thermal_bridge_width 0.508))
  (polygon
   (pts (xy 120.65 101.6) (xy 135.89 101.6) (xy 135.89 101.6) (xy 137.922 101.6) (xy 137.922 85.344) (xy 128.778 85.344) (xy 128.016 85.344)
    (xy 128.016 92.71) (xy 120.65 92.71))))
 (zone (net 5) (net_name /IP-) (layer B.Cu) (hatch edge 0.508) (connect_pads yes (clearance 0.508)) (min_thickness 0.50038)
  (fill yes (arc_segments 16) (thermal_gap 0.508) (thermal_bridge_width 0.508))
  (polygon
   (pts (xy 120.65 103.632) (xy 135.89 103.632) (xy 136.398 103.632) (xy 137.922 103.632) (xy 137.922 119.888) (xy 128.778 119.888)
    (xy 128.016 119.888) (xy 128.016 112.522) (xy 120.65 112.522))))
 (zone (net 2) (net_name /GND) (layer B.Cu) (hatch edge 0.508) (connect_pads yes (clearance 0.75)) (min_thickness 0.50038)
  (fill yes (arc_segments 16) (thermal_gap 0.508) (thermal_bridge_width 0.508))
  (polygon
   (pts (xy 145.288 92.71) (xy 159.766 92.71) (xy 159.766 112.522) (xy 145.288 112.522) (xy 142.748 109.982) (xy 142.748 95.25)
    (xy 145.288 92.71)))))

